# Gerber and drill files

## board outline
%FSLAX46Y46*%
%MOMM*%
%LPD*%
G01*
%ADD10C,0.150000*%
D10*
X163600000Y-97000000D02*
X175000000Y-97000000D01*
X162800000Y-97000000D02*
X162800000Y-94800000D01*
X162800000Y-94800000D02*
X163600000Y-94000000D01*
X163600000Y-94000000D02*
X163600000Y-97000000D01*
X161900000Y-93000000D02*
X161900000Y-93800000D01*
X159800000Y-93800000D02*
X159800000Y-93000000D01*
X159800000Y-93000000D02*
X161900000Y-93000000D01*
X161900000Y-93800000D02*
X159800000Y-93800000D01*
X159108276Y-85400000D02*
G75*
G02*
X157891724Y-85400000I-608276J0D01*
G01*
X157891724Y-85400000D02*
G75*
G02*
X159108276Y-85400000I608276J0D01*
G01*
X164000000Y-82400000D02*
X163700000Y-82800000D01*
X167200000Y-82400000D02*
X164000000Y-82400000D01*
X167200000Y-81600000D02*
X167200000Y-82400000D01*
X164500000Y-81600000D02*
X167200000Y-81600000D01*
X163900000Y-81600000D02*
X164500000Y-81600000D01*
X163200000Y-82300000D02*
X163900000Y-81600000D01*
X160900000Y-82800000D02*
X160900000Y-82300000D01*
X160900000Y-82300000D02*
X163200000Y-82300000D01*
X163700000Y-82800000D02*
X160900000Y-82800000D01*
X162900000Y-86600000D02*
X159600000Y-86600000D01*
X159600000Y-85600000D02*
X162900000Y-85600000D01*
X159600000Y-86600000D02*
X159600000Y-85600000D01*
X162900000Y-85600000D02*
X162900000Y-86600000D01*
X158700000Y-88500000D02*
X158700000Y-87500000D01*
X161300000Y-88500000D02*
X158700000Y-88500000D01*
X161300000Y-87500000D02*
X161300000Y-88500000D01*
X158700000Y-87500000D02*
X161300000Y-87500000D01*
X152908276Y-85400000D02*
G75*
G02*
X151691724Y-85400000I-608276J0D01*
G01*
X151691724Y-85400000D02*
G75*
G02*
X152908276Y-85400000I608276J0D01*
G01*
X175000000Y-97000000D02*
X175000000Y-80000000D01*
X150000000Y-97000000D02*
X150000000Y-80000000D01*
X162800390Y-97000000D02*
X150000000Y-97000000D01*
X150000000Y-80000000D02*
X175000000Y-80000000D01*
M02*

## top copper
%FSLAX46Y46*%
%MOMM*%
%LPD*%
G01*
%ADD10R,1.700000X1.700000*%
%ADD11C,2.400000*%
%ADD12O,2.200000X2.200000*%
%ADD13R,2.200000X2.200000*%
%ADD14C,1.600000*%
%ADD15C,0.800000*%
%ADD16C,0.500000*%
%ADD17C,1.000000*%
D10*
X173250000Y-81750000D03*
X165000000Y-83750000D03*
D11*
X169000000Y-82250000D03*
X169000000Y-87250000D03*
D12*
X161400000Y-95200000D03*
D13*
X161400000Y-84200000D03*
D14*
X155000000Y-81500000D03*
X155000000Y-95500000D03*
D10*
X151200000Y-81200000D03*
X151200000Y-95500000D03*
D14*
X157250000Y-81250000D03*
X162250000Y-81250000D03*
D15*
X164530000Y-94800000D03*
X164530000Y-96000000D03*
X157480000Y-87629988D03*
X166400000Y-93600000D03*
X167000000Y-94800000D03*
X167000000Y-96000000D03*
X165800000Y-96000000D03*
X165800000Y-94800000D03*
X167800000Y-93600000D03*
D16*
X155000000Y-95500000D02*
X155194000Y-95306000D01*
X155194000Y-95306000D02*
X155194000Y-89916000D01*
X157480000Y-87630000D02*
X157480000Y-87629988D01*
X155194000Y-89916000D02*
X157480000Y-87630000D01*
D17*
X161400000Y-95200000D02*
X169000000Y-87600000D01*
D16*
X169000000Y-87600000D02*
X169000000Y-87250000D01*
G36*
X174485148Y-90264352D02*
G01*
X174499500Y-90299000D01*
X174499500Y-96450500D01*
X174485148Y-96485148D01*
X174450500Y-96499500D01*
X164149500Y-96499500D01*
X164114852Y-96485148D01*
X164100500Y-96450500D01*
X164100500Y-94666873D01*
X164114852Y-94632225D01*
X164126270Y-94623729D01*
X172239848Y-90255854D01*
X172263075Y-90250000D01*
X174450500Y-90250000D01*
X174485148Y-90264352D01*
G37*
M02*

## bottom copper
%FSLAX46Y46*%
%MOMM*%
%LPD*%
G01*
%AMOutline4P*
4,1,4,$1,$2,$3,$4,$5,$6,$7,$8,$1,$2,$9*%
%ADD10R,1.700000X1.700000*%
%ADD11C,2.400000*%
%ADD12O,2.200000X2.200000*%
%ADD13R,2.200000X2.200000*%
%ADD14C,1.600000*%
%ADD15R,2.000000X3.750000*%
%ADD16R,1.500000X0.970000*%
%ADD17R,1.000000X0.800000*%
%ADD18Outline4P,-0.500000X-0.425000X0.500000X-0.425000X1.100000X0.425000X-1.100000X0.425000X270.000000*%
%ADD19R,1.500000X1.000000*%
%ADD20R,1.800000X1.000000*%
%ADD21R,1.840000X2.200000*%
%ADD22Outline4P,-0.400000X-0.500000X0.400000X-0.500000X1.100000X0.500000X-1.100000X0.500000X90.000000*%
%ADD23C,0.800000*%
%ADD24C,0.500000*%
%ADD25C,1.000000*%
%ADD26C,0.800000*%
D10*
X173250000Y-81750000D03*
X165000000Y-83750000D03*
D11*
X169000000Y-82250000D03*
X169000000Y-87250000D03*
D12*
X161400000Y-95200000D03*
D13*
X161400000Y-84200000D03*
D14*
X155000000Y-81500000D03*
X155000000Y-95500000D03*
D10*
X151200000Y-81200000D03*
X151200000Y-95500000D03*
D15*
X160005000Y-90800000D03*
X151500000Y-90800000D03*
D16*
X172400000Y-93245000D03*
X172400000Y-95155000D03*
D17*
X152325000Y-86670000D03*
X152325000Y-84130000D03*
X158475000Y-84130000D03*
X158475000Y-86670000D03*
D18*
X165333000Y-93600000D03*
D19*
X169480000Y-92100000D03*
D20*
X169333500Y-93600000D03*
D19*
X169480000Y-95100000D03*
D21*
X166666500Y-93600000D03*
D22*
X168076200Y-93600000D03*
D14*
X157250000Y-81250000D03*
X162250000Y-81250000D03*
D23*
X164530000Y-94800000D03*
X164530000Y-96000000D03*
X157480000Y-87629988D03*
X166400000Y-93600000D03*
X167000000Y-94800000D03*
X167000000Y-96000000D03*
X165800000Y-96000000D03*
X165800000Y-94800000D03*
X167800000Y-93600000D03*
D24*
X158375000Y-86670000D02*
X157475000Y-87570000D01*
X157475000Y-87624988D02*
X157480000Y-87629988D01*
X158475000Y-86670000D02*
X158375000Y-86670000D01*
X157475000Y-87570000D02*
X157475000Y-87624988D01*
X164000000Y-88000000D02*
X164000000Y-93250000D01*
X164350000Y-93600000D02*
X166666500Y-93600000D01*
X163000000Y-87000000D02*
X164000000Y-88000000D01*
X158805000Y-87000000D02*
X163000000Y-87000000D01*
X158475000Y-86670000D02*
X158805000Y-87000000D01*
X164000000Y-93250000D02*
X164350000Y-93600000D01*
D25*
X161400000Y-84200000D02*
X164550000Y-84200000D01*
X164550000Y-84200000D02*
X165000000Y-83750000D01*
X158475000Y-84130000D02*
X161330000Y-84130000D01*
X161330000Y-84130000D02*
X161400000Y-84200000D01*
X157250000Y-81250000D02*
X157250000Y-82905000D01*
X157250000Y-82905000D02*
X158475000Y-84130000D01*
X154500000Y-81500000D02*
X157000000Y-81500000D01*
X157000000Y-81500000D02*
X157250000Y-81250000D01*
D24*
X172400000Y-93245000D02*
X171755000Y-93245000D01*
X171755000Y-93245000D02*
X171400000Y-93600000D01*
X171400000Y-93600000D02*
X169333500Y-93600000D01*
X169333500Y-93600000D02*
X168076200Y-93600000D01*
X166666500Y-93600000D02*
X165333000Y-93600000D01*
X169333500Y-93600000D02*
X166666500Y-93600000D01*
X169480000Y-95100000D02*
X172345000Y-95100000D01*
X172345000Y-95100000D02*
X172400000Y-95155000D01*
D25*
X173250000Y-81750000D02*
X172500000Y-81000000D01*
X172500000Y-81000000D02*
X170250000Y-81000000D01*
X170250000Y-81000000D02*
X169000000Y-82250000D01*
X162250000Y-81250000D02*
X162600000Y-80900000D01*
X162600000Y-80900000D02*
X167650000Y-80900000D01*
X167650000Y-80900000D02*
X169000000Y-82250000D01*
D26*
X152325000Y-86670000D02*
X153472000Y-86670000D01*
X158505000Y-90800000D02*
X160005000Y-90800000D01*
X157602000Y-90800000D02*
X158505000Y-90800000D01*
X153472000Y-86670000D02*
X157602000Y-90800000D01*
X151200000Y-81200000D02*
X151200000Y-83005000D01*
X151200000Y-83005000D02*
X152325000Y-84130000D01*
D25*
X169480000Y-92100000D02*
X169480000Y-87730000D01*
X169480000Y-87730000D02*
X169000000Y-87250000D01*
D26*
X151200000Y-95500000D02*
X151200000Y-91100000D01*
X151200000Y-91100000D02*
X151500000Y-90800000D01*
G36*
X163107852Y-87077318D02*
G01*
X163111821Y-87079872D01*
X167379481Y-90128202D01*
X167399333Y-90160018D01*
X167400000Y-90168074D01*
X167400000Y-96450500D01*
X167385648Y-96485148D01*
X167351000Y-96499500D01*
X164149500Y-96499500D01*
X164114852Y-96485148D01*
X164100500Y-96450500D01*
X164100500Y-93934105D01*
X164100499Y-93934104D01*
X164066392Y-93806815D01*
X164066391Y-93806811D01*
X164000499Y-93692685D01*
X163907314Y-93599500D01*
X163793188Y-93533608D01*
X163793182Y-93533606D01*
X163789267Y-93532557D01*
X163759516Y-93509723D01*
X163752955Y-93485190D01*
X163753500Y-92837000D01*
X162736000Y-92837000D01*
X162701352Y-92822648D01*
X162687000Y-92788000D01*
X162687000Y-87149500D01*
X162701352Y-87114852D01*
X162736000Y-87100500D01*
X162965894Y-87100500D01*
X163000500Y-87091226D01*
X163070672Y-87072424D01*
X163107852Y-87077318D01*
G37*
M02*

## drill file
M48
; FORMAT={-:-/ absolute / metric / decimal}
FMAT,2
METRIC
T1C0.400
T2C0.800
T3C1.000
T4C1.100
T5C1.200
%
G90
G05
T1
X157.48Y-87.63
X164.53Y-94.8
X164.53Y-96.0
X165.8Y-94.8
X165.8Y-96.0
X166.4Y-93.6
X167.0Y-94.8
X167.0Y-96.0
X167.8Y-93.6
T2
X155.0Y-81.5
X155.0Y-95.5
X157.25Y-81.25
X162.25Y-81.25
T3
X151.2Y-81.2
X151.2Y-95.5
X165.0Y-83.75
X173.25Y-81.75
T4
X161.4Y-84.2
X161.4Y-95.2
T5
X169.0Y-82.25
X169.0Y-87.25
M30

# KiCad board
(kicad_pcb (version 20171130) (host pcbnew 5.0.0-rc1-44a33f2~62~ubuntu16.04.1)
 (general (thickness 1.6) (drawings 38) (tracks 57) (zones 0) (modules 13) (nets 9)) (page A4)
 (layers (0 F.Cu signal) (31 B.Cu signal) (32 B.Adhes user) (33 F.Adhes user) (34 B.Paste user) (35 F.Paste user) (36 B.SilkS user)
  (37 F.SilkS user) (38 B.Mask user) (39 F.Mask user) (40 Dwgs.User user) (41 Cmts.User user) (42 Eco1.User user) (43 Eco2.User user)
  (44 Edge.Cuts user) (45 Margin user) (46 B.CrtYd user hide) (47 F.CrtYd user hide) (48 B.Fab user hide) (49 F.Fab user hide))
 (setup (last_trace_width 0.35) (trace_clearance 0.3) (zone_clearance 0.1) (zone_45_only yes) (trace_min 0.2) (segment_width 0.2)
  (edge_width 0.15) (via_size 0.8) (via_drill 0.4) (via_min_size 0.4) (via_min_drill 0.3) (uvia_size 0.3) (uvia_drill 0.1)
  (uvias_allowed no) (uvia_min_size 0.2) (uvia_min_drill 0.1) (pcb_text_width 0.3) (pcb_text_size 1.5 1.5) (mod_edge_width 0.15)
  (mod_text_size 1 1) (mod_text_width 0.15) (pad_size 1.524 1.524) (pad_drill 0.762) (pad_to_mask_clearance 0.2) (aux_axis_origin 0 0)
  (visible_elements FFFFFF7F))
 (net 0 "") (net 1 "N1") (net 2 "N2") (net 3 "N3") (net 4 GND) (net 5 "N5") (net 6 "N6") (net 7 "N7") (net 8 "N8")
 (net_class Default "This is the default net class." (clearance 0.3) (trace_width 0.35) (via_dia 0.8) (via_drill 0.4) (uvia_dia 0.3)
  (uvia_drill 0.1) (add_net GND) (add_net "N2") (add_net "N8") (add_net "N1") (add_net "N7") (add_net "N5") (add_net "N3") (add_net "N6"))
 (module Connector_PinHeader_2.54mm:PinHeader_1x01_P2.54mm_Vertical (layer F.Cu) (at 173.25 81.75)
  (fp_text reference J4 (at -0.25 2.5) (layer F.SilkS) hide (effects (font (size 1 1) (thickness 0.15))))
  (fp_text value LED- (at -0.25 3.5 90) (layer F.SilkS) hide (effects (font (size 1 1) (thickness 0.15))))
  (pad 1 thru_hole rect (at 0 0) (size 1.7 1.7) (drill 1) (layers *.Cu *.Mask) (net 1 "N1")))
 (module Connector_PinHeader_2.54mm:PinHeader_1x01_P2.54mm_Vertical (layer F.Cu) (at 165 83.75)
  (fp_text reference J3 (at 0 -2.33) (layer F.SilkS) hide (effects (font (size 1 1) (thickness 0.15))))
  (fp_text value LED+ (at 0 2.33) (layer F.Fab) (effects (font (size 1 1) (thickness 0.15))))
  (pad 1 thru_hole rect (at 0 0) (size 1.7 1.7) (drill 1) (layers *.Cu *.Mask) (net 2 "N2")))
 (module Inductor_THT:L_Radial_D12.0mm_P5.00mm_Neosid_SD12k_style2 (layer F.Cu) (at 169 82.25 270)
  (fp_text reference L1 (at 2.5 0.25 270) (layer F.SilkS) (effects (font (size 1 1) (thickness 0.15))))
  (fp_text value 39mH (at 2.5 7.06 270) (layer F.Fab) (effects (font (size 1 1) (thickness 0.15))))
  (pad 1 thru_hole circle (at 0 0 270) (size 2.4 2.4) (drill 1.2) (layers *.Cu *.Mask) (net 1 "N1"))
  (pad 2 thru_hole circle (at 5 0 270) (size 2.4 2.4) (drill 1.2) (layers *.Cu *.Mask) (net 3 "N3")))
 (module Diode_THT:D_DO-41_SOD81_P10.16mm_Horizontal (layer F.Cu) (at 161.4 84.2 270)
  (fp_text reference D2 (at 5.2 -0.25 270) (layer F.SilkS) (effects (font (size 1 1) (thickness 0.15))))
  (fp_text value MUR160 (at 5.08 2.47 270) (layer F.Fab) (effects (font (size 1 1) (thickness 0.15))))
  (pad 2 thru_hole oval (at 11 0 270) (size 2.2 2.2) (drill 1.1) (layers *.Cu *.Mask) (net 3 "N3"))
  (pad 1 thru_hole rect (at 0 0 270) (size 2.2 2.2) (drill 1.1) (layers *.Cu *.Mask) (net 2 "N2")))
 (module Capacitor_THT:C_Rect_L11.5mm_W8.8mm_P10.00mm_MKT (layer F.Cu) (at 155 83.5 270)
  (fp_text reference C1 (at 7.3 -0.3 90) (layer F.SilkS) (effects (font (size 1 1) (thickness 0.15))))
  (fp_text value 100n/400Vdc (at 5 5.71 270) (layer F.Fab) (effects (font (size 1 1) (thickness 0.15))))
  (pad 1 thru_hole circle (at -2 0 270) (size 1.6 1.6) (drill 0.8) (layers *.Cu *.Mask) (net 2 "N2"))
  (pad 2 thru_hole circle (at 12 0 270) (size 1.6 1.6) (drill 0.8) (layers *.Cu *.Mask) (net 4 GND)))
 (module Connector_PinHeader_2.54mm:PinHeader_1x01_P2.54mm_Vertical (layer F.Cu) (at 151.2 81.2)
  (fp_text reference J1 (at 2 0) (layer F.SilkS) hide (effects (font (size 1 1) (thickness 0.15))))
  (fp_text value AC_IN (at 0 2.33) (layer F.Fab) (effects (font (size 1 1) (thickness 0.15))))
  (pad 1 thru_hole rect (at 0 0) (size 1.7 1.7) (drill 1) (layers *.Cu *.Mask) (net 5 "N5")))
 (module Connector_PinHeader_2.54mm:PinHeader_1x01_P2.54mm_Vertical (layer F.Cu) (at 151.2 95.5)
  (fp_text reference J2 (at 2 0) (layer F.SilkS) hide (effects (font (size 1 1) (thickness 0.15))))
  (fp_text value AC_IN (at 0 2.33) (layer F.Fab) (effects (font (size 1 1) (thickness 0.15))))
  (pad 1 thru_hole rect (at 0 0) (size 1.7 1.7) (drill 1) (layers *.Cu *.Mask) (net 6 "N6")))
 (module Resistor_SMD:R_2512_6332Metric (layer B.Cu) (at 157 90.8 180)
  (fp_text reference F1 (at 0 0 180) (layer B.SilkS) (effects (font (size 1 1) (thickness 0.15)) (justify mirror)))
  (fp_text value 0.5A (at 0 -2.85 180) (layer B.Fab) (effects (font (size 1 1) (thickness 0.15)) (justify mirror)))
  (pad 1 smd rect (at -3.005 0 180) (size 2 3.75) (layers B.Cu B.Paste B.Mask) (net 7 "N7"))
  (pad 2 smd rect (at 5.5 0 180) (size 2 3.75) (layers B.Cu B.Paste B.Mask) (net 6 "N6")))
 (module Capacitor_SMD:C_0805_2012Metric (layer B.Cu) (at 172.4 94.2 270)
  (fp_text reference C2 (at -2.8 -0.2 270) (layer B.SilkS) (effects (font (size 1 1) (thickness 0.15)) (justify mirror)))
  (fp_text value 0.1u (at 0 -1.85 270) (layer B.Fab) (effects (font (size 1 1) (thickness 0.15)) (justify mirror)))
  (pad 1 smd rect (at -0.955 0 270) (size 0.97 1.5) (layers B.Cu B.Paste B.Mask) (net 4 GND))
  (pad 2 smd rect (at 0.955 0 270) (size 0.97 1.5) (layers B.Cu B.Paste B.Mask) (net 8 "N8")))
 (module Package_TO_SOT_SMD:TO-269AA (layer B.Cu) (at 155.4 85.4)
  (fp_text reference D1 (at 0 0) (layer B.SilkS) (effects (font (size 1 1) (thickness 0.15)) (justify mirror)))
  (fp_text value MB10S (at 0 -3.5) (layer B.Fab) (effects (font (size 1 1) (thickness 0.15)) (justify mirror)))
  (pad 1 smd rect (at -3.075 1.27) (size 1 0.8) (layers B.Cu B.Paste B.Mask) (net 7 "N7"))
  (pad 2 smd rect (at -3.075 -1.27) (size 1 0.8) (layers B.Cu B.Paste B.Mask) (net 5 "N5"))
  (pad 3 smd rect (at 3.075 -1.27) (size 1 0.8) (layers B.Cu B.Paste B.Mask) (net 2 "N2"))
  (pad 4 smd rect (at 3.075 1.27) (size 1 0.8) (layers B.Cu B.Paste B.Mask) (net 4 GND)))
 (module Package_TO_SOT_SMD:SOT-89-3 (layer B.Cu) (at 168 93.6 180)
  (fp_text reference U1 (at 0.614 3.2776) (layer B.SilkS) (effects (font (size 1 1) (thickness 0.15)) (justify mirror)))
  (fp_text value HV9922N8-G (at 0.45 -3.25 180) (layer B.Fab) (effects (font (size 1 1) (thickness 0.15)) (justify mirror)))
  (pad 2 smd trapezoid (at 2.667 0 270) (size 1.6 0.85) (rect_delta 0 -0.6) (layers B.Cu B.Paste B.Mask) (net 4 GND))
  (pad 1 smd rect (at -1.48 1.5 270) (size 1 1.5) (layers B.Cu B.Paste B.Mask) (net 3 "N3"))
  (pad 2 smd rect (at -1.3335 0 270) (size 1 1.8) (layers B.Cu B.Paste B.Mask) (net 4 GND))
  (pad 3 smd rect (at -1.48 -1.5 270) (size 1 1.5) (layers B.Cu B.Paste B.Mask) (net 8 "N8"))
  (pad 2 smd rect (at 1.3335 0 270) (size 2.2 1.84) (layers B.Cu B.Paste B.Mask) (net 4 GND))
  (pad 2 smd trapezoid (at -0.0762 0 90) (size 1.5 1) (rect_delta 0 -0.7) (layers B.Cu B.Paste B.Mask) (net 4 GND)))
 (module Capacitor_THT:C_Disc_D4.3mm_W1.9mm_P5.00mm (layer F.Cu) (at 157.25 81.25)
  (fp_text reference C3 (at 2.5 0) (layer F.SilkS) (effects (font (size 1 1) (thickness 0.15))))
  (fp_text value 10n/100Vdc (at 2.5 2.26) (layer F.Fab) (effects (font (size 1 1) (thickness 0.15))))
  (pad 1 thru_hole circle (at 0 0) (size 1.6 1.6) (drill 0.8) (layers *.Cu *.Mask) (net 2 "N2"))
  (pad 2 thru_hole circle (at 5 0) (size 1.6 1.6) (drill 0.8) (layers *.Cu *.Mask) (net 1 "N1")))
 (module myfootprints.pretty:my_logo (layer F.Cu) (at 170.942 93.98)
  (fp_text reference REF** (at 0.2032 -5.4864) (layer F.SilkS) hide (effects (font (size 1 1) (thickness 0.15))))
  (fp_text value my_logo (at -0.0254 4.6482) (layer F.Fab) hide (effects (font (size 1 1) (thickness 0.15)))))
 (gr_line (start 163.6 97) (end 175 97) (layer Edge.Cuts) (width 0.15))
 (gr_line (start 162.8 97) (end 162.8 94.8) (layer Edge.Cuts) (width 0.15))
 (gr_line (start 162.8 94.8) (end 163.6 94) (layer Edge.Cuts) (width 0.15))
 (gr_line (start 163.6 94) (end 163.6 97) (layer Edge.Cuts) (width 0.15))
 (gr_line (start 161.9 93) (end 161.9 93.8) (layer Edge.Cuts) (width 0.15))
 (gr_line (start 159.8 93.8) (end 159.8 93) (layer Edge.Cuts) (width 0.15))
 (gr_line (start 159.8 93) (end 161.9 93) (layer Edge.Cuts) (width 0.15))
 (gr_line (start 161.9 93.8) (end 159.8 93.8) (layer Edge.Cuts) (width 0.15))
 (gr_circle (center 158.5 85.4) (end 159.108276 85.4) (layer Edge.Cuts) (width 0.15))
 (gr_line (start 164 82.4) (end 163.7 82.8) (layer Edge.Cuts) (width 0.15))
 (gr_line (start 167.2 82.4) (end 164 82.4) (layer Edge.Cuts) (width 0.15))
 (gr_line (start 167.2 81.6) (end 167.2 82.4) (layer Edge.Cuts) (width 0.15))
 (gr_line (start 164.5 81.6) (end 167.2 81.6) (layer Edge.Cuts) (width 0.15))
 (gr_line (start 163.9 81.6) (end 164.5 81.6) (layer Edge.Cuts) (width 0.15))
 (gr_line (start 163.2 82.3) (end 163.9 81.6) (layer Edge.Cuts) (width 0.15))
 (gr_line (start 160.9 82.8) (end 160.9 82.3) (layer Edge.Cuts) (width 0.15))
 (gr_line (start 160.9 82.3) (end 163.2 82.3) (layer Edge.Cuts) (width 0.15))
 (gr_line (start 163.7 82.8) (end 160.9 82.8) (layer Edge.Cuts) (width 0.15))
 (gr_line (start 162.9 86.6) (end 159.6 86.6) (layer Edge.Cuts) (width 0.15))
 (gr_line (start 159.6 85.6) (end 162.9 85.6) (layer Edge.Cuts) (width 0.15))
 (gr_line (start 159.6 86.6) (end 159.6 85.6) (layer Edge.Cuts) (width 0.15))
 (gr_line (start 162.9 85.6) (end 162.9 86.6) (layer Edge.Cuts) (width 0.15))
 (gr_line (start 158.7 88.5) (end 158.7 87.5) (layer Edge.Cuts) (width 0.15))
 (gr_line (start 161.3 88.5) (end 158.7 88.5) (layer Edge.Cuts) (width 0.15))
 (gr_line (start 161.3 87.5) (end 161.3 88.5) (layer Edge.Cuts) (width 0.15))
 (gr_line (start 158.7 87.5) (end 161.3 87.5) (layer Edge.Cuts) (width 0.15))
 (gr_circle (center 152.3 85.4) (end 152.908276 85.4) (layer Edge.Cuts) (width 0.15))
 (gr_line (start 175 97) (end 175 80) (layer Edge.Cuts) (width 0.15))
 (gr_line (start 150 97) (end 150 80) (layer Edge.Cuts) (width 0.15))
 (gr_line (start 162.80039 97) (end 150 97) (layer Edge.Cuts) (width 0.15))
 (gr_line (start 150 80) (end 175 80) (layer Edge.Cuts) (width 0.15))
 (via (at 164.53 94.8) (size 0.8) (drill 0.4) (layers F.Cu B.Cu) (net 4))
 (via (at 164.53 96) (size 0.8) (drill 0.4) (layers F.Cu B.Cu) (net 4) (status 1000000))
 (segment (start 155 95.5) (end 155.194 95.306) (width 0.5) (layer F.Cu) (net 4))
 (segment (start 155.194 95.306) (end 155.194 89.916) (width 0.5) (layer F.Cu) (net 4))
 (segment (start 157.48 87.63) (end 157.48 87.629988) (width 0.5) (layer F.Cu) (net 4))
 (segment (start 155.194 89.916) (end 157.48 87.63) (width 0.5) (layer F.Cu) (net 4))
 (segment (start 158.375 86.67) (end 157.475 87.57) (width 0.5) (layer B.Cu) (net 4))
 (segment (start 157.475 87.624988) (end 157.48 87.629988) (width 0.5) (layer B.Cu) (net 4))
 (segment (start 158.475 86.67) (end 158.375 86.67) (width 0.5) (layer B.Cu) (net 4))
 (segment (start 157.475 87.57) (end 157.475 87.624988) (width 0.5) (layer B.Cu) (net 4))
 (via (at 157.48 87.629988) (size 0.8) (drill 0.4) (layers F.Cu B.Cu) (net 4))
 (segment (start 164 88) (end 164 93.25) (width 0.5) (layer B.Cu) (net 4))
 (segment (start 164.35 93.6) (end 166.6665 93.6) (width 0.5) (layer B.Cu) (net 4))
 (segment (start 163 87) (end 164 88) (width 0.5) (layer B.Cu) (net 4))
 (segment (start 158.805 87) (end 163 87) (width 0.5) (layer B.Cu) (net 4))
 (segment (start 158.475 86.67) (end 158.805 87) (width 0.5) (layer B.Cu) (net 4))
 (segment (start 164 93.25) (end 164.35 93.6) (width 0.5) (layer B.Cu) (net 4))
 (via (at 166.4 93.6) (size 0.8) (drill 0.4) (layers F.Cu B.Cu) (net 4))
 (via (at 167 94.8) (size 0.8) (drill 0.4) (layers F.Cu B.Cu) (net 4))
 (via (at 167 96) (size 0.8) (drill 0.4) (layers F.Cu B.Cu) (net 4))
 (via (at 165.8 96) (size 0.8) (drill 0.4) (layers F.Cu B.Cu) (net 4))
 (via (at 165.8 94.8) (size 0.8) (drill 0.4) (layers F.Cu B.Cu) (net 4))
 (via (at 167.8 93.6) (size 0.8) (drill 0.4) (layers F.Cu B.Cu) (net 4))
 (segment (start 161.4 84.2) (end 164.55 84.2) (width 1) (layer B.Cu) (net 2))
 (segment (start 164.55 84.2) (end 165 83.75) (width 1) (layer B.Cu) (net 2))
 (segment (start 158.475 84.13) (end 161.33 84.13) (width 1) (layer B.Cu) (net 2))
 (segment (start 161.33 84.13) (end 161.4 84.2) (width 1) (layer B.Cu) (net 2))
 (segment (start 157.25 81.25) (end 157.25 82.905) (width 1) (layer B.Cu) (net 2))
 (segment (start 157.25 82.905) (end 158.475 84.13) (width 1) (layer B.Cu) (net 2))
 (segment (start 154.5 81.5) (end 157 81.5) (width 1) (layer B.Cu) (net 2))
 (segment (start 157 81.5) (end 157.25 81.25) (width 1) (layer B.Cu) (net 2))
 (segment (start 172.4 93.245) (end 171.755 93.245) (width 0.5) (layer B.Cu) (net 4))
 (segment (start 171.755 93.245) (end 171.4 93.6) (width 0.5) (layer B.Cu) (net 4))
 (segment (start 171.4 93.6) (end 169.3335 93.6) (width 0.5) (layer B.Cu) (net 4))
 (segment (start 169.3335 93.6) (end 168.0762 93.6) (width 0.5) (layer B.Cu) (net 4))
 (segment (start 166.6665 93.6) (end 165.333 93.6) (width 0.5) (layer B.Cu) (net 4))
 (segment (start 169.3335 93.6) (end 166.6665 93.6) (width 0.5) (layer B.Cu) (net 4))
 (segment (start 169.48 95.1) (end 172.345 95.1) (width 0.5) (layer B.Cu) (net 8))
 (segment (start 172.345 95.1) (end 172.4 95.155) (width 0.5) (layer B.Cu) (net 8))
 (segment (start 173.25 81.75) (end 172.5 81) (width 1) (layer B.Cu) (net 1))
 (segment (start 172.5 81) (end 170.25 81) (width 1) (layer B.Cu) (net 1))
 (segment (start 170.25 81) (end 169 82.25) (width 1) (layer B.Cu) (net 1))
 (segment (start 162.25 81.25) (end 162.6 80.9) (width 1) (layer B.Cu) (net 1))
 (segment (start 162.6 80.9) (end 167.65 80.9) (width 1) (layer B.Cu) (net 1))
 (segment (start 167.65 80.9) (end 169 82.25) (width 1) (layer B.Cu) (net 1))
 (segment (start 152.325 86.67) (end 153.472 86.67) (width 0.8) (layer B.Cu) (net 7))
 (segment (start 158.505 90.8) (end 160.005 90.8) (width 0.8) (layer B.Cu) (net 7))
 (segment (start 157.602 90.8) (end 158.505 90.8) (width 0.8) (layer B.Cu) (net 7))
 (segment (start 153.472 86.67) (end 157.602 90.8) (width 0.8) (layer B.Cu) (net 7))
 (segment (start 151.2 81.2) (end 151.2 83.005) (width 0.8) (layer B.Cu) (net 5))
 (segment (start 151.2 83.005) (end 152.325 84.13) (width 0.8) (layer B.Cu) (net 5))
 (segment (start 169.48 92.1) (end 169.48 87.73) (width 1) (layer B.Cu) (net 3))
 (segment (start 169.48 87.73) (end 169 87.25) (width 1) (layer B.Cu) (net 3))
 (segment (start 161.4 95.2) (end 169 87.6) (width 1) (layer F.Cu) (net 3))
 (segment (start 169 87.6) (end 169 87.25) (width 0.5) (layer F.Cu) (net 3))
 (segment (start 151.2 95.5) (end 151.2 91.1) (width 0.8) (layer B.Cu) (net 6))
 (segment (start 151.2 91.1) (end 151.5 90.8) (width 0.8) (layer B.Cu) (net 6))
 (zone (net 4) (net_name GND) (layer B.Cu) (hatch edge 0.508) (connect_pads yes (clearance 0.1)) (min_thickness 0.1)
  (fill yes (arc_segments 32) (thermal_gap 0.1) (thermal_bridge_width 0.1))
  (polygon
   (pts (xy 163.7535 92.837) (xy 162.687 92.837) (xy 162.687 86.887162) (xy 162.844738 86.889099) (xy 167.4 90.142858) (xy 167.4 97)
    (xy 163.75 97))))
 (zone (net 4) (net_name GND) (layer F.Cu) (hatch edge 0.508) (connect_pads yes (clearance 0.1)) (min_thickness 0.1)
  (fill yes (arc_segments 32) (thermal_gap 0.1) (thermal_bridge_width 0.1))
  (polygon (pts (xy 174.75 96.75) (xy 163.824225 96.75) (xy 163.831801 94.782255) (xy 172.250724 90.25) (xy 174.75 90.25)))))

